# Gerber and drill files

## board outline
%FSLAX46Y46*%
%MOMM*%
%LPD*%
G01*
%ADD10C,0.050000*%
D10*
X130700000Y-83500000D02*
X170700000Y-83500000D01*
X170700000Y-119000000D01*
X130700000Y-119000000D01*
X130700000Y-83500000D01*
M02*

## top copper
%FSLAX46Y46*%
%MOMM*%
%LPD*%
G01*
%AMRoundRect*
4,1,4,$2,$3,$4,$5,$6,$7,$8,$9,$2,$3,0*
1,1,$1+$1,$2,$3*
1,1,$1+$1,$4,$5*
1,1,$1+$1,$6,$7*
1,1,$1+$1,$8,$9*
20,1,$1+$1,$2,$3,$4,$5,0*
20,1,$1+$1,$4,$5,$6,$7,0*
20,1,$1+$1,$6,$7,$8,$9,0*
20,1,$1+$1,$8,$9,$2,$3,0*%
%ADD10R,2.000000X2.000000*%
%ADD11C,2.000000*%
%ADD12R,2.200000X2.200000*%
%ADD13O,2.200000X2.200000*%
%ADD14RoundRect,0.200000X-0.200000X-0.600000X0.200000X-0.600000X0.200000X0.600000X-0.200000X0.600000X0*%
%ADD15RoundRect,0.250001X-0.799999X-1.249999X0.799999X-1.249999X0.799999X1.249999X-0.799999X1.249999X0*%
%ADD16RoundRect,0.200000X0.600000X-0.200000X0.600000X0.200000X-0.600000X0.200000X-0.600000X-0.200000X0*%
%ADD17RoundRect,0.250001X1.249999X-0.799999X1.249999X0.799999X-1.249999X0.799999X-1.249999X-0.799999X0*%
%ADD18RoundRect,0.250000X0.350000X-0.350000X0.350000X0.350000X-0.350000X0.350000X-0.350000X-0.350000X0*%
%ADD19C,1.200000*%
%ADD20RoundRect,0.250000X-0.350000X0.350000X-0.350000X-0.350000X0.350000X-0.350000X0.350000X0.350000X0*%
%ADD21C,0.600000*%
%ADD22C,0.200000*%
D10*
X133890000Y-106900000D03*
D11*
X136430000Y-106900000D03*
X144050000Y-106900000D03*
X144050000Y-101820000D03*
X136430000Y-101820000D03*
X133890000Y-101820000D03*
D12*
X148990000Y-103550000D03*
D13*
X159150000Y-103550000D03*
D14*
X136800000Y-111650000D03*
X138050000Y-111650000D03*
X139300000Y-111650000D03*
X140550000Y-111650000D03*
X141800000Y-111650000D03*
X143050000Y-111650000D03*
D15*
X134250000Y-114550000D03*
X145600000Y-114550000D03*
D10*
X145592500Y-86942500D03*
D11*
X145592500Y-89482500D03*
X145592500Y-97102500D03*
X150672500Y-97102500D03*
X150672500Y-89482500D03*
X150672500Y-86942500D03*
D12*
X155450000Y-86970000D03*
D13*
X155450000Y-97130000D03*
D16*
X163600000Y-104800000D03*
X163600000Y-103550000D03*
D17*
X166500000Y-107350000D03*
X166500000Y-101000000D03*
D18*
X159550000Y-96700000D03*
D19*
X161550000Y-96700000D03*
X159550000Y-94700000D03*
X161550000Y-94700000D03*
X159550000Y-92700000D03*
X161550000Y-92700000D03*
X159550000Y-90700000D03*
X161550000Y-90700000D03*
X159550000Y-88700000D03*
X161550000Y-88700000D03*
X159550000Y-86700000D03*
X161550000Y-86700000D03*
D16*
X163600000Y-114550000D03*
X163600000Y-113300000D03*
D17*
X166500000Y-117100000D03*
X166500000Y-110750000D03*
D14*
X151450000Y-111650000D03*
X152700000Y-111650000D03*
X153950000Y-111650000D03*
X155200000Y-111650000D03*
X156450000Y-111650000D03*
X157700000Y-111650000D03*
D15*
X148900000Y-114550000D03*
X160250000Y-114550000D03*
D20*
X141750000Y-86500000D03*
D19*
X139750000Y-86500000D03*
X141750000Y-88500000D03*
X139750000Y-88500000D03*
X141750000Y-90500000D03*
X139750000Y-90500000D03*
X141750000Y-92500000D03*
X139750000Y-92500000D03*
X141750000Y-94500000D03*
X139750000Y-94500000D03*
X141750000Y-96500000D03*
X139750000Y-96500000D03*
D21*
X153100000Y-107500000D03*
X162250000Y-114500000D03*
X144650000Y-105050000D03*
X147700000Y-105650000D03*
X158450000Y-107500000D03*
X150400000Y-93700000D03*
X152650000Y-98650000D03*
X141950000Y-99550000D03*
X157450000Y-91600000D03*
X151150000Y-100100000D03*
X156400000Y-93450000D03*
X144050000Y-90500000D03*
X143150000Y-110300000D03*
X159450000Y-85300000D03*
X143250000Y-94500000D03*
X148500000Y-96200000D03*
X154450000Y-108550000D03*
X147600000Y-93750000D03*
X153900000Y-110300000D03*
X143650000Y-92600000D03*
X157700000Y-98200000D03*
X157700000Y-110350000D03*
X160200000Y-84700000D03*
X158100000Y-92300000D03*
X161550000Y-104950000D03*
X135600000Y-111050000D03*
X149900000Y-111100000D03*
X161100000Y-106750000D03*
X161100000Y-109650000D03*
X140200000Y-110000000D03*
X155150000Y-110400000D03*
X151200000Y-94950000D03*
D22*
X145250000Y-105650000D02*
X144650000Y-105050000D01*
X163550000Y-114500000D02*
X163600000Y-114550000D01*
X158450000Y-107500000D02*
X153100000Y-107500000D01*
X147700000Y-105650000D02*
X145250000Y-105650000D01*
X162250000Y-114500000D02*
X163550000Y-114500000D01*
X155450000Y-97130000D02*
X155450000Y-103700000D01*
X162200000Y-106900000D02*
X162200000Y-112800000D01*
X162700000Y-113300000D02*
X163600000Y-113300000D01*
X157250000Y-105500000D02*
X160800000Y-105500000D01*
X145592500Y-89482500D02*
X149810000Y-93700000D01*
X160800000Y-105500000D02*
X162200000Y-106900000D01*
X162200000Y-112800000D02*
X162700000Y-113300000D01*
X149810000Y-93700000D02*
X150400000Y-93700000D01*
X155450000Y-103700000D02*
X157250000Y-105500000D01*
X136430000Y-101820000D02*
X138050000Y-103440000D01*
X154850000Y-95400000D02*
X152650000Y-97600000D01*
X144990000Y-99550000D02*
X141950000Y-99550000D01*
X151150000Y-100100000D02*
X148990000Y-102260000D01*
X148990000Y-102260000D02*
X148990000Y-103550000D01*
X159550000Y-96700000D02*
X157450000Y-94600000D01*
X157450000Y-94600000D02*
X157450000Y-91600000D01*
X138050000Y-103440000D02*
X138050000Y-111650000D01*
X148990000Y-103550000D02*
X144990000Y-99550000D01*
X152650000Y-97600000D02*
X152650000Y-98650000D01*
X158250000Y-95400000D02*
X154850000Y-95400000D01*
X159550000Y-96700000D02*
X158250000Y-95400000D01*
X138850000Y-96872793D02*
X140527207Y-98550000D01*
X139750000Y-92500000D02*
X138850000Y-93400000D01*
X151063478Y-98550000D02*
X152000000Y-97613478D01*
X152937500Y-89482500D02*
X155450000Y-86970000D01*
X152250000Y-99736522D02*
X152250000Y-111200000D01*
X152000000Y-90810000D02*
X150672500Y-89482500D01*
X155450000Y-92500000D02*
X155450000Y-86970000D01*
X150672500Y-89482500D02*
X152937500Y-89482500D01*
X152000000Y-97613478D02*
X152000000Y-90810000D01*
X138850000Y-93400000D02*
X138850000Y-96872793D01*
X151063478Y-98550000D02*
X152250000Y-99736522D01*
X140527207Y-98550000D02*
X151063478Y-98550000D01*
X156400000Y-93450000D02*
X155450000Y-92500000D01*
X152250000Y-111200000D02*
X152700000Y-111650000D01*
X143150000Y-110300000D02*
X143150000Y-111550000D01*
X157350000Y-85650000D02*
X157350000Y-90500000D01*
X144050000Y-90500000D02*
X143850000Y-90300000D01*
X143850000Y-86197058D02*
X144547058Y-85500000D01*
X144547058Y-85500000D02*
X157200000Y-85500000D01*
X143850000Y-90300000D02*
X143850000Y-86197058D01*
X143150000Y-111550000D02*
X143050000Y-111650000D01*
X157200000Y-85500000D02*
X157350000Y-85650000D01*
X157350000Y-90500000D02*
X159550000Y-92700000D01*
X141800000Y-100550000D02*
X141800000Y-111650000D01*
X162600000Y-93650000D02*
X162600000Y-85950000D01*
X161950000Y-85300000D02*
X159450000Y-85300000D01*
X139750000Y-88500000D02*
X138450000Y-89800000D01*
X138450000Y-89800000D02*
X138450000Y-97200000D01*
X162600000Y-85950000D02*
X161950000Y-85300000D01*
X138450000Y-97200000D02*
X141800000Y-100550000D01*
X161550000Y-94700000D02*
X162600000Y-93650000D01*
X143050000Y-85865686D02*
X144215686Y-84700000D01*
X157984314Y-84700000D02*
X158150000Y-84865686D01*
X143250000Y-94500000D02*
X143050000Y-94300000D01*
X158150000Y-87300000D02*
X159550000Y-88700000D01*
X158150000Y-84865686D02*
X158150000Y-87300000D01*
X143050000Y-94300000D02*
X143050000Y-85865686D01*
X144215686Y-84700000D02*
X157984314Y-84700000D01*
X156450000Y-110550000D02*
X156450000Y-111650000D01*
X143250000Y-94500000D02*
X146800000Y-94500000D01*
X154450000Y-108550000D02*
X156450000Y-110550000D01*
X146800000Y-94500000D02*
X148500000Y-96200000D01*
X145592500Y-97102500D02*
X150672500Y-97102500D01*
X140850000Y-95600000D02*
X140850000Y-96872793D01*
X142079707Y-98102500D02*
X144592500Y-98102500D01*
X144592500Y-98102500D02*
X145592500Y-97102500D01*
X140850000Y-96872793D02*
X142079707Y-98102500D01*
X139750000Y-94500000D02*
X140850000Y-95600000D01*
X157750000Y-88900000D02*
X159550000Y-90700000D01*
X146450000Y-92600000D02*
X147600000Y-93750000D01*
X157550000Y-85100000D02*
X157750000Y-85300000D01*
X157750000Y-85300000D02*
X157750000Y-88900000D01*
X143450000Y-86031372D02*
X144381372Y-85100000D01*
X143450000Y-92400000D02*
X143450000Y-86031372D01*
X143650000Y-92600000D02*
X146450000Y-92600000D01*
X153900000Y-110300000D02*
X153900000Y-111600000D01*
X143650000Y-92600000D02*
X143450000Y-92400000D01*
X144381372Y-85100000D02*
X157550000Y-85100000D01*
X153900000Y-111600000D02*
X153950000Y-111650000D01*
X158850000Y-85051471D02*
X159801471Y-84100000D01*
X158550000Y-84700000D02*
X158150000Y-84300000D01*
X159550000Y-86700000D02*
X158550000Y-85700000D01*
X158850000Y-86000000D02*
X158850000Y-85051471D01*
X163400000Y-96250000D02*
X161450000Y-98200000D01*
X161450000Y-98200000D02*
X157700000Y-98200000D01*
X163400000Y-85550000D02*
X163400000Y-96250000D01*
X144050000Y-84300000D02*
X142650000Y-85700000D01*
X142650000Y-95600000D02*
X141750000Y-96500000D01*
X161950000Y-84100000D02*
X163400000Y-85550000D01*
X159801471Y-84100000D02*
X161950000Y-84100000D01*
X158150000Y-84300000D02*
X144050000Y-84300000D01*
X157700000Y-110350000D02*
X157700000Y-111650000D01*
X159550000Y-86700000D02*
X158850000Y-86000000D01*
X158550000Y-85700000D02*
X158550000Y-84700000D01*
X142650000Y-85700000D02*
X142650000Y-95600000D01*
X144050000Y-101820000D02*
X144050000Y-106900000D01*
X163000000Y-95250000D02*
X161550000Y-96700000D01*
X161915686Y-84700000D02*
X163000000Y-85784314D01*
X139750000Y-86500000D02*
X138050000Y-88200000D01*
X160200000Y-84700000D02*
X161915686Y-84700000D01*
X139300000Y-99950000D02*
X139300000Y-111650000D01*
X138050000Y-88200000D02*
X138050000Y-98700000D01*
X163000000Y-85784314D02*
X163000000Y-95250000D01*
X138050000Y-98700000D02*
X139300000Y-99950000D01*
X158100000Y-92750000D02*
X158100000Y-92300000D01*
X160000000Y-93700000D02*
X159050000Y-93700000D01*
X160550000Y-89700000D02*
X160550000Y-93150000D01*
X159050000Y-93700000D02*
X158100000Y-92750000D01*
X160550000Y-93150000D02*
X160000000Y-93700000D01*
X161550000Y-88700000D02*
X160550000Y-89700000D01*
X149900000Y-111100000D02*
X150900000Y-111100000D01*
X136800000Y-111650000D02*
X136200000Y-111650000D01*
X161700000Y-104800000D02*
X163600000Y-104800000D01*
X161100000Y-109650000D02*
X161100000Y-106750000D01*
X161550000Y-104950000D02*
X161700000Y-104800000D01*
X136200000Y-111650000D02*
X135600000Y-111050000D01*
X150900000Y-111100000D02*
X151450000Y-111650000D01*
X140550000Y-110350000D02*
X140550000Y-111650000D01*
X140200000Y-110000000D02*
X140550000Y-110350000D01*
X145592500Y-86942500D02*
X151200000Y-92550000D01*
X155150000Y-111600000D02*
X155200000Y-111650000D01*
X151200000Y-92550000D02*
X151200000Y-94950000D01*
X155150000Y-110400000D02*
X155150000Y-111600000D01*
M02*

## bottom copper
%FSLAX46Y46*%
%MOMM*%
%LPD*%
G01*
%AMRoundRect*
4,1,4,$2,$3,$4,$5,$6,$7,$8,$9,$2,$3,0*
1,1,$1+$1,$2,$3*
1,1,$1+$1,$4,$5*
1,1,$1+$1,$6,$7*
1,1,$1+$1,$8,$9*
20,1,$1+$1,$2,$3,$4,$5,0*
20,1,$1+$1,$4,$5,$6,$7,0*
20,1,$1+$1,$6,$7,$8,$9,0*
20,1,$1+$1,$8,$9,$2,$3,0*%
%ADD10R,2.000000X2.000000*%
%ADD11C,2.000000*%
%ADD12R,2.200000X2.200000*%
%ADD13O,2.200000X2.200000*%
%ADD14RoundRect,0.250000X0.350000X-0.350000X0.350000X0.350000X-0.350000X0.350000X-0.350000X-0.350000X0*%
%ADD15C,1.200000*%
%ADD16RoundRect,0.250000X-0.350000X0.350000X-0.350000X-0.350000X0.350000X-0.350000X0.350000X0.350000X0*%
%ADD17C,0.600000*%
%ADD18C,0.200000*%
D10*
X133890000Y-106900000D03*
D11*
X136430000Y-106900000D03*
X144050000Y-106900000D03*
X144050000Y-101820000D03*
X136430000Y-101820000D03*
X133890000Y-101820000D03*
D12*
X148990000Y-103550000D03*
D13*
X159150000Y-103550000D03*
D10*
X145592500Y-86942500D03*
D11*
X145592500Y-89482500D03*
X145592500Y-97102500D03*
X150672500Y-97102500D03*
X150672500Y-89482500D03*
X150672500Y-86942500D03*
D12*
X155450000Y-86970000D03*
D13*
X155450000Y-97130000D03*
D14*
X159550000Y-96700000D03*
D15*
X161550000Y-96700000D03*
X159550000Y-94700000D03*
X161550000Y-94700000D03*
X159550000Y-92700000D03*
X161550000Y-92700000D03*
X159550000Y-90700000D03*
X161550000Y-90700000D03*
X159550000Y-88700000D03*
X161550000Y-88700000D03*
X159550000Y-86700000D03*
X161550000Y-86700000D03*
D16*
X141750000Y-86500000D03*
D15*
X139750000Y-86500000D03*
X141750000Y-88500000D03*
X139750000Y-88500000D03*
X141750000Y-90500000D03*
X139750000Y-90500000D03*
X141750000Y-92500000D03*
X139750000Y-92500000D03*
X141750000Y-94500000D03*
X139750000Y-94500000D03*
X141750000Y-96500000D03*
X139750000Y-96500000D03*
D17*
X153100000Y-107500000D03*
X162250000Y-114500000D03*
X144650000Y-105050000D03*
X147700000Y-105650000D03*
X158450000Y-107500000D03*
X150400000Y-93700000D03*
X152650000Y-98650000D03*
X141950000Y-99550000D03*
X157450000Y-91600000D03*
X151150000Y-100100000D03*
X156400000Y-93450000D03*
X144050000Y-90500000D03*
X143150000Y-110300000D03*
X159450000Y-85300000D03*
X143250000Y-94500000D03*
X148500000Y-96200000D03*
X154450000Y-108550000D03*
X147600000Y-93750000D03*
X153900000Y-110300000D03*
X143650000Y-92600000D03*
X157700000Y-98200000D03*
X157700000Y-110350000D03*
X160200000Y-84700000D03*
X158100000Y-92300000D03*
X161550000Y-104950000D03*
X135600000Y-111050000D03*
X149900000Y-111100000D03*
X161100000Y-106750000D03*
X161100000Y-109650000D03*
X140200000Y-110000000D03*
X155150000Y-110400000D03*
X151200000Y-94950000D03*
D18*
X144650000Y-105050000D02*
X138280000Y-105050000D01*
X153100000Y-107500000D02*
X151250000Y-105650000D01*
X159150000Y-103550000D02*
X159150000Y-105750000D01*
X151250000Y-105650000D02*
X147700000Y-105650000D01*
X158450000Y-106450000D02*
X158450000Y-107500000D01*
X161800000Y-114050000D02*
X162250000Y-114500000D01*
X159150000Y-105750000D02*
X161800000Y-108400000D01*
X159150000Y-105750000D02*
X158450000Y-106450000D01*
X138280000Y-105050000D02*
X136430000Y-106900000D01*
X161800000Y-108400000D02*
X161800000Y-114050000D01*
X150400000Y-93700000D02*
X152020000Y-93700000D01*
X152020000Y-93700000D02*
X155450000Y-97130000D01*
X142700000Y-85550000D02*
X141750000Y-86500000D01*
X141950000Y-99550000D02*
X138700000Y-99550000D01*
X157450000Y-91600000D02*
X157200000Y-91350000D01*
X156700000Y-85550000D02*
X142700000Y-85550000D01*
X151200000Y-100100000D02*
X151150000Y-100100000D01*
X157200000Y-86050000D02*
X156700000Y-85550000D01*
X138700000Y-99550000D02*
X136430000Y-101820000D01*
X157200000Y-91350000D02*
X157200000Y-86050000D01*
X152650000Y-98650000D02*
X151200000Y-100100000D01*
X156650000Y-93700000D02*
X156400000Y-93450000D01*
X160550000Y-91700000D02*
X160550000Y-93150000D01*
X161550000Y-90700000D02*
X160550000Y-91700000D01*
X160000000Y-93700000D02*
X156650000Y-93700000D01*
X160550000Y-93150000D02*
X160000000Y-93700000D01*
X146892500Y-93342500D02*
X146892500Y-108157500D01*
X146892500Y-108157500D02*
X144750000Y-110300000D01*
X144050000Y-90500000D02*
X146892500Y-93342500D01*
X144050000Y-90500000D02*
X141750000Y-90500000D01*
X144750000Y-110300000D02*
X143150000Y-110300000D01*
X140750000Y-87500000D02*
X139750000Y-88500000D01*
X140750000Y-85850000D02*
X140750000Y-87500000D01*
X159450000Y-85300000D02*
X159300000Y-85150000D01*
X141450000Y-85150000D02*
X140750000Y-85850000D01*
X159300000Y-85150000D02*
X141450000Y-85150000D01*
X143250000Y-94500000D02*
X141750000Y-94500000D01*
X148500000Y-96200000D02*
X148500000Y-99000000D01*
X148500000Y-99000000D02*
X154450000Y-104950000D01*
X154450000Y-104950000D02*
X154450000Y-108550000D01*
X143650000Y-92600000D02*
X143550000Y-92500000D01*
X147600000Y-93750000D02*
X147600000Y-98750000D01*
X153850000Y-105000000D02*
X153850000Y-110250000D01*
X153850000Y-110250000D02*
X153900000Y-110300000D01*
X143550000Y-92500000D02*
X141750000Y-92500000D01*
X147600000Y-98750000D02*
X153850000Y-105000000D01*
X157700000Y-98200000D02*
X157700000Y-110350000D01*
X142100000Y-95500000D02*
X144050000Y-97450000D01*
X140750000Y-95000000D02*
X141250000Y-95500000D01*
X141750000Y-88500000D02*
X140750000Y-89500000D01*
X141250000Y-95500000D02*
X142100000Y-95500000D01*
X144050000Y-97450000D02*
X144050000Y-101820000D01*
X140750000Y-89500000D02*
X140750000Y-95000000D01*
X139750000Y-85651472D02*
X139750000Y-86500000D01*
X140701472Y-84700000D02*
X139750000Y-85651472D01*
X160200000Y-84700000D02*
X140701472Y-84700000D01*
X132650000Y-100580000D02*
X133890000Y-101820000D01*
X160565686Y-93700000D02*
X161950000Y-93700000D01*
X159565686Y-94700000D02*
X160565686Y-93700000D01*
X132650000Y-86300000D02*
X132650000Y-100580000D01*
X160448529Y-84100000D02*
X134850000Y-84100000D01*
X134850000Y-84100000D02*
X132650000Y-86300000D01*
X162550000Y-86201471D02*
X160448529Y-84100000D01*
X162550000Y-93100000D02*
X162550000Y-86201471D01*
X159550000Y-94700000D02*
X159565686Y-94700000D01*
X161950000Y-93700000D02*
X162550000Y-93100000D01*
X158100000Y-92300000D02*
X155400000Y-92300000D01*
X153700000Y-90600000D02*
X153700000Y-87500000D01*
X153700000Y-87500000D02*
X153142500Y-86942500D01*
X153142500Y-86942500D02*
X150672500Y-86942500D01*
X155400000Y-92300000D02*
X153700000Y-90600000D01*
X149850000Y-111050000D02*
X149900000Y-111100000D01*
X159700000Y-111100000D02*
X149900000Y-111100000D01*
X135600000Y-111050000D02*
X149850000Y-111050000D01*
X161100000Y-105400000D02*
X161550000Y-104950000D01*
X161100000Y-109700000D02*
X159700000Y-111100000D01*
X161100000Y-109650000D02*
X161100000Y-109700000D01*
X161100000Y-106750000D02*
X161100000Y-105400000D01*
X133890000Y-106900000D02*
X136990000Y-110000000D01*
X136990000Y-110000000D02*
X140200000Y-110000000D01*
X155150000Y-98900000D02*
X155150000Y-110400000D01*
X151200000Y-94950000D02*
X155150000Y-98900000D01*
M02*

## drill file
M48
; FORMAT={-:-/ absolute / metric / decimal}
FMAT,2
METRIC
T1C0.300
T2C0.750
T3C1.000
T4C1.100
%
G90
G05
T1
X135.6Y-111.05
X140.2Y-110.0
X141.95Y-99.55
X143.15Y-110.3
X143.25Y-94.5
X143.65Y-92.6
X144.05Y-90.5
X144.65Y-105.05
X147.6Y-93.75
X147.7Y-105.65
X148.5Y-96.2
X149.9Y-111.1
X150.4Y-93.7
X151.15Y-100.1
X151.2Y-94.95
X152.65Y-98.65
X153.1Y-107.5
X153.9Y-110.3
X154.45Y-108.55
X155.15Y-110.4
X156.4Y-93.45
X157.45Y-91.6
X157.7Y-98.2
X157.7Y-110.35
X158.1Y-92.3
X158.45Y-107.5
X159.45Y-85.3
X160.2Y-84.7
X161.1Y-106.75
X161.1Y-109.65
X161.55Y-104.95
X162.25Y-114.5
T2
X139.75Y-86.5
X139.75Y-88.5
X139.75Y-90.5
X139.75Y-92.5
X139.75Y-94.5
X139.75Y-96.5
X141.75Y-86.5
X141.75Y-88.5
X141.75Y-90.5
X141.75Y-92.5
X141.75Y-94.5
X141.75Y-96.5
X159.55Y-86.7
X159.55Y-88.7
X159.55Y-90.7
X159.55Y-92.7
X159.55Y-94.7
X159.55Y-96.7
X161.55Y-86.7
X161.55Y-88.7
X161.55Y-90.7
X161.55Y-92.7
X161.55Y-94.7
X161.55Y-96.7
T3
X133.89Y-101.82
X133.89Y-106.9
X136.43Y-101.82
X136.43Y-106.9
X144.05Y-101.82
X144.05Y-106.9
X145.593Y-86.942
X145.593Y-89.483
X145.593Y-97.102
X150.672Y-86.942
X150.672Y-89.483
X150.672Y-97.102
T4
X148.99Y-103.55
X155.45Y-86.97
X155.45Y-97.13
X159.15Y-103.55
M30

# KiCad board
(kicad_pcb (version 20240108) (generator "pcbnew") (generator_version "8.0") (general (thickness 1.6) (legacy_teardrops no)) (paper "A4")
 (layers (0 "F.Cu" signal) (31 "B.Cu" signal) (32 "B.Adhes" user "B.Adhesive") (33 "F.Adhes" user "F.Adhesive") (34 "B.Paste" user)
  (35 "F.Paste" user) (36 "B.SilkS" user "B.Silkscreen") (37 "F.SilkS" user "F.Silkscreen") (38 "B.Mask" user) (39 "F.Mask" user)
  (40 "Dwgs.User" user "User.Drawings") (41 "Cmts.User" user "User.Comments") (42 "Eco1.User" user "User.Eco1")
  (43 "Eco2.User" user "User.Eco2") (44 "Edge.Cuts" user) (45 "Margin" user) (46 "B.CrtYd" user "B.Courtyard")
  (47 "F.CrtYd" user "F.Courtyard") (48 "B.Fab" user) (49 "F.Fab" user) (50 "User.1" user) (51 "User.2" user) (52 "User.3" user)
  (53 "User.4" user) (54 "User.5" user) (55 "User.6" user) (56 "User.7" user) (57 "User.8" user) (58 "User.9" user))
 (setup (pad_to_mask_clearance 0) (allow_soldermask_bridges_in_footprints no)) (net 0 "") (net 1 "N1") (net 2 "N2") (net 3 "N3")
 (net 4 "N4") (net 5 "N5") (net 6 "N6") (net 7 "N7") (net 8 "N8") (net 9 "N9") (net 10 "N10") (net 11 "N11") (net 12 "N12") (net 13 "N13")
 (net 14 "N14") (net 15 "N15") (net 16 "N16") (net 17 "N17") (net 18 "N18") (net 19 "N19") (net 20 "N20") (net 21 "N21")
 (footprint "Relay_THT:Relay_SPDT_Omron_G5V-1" (layer "F.Cu") (at 133.89 106.9 90)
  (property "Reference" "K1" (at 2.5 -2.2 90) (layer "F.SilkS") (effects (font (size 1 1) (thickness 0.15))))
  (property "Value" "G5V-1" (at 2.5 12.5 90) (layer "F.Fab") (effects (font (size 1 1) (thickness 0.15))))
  (pad "1" thru_hole rect (at 0 0 90) (size 2 2) (drill 1) (layers "*.Cu" "*.Mask") (remove_unused_layers no) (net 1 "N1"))
  (pad "2" thru_hole circle (at 0 2.54 90) (size 2 2) (drill 1) (layers "*.Cu" "*.Mask") (remove_unused_layers no) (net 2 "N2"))
  (pad "5" thru_hole circle (at 0 10.16 90) (size 2 2) (drill 1) (layers "*.Cu" "*.Mask") (remove_unused_layers no) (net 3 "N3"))
  (pad "6" thru_hole circle (at 5.08 10.16 90) (size 2 2) (drill 1) (layers "*.Cu" "*.Mask") (remove_unused_layers no) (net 3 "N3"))
  (pad "9" thru_hole circle (at 5.08 2.54 90) (size 2 2) (drill 1) (layers "*.Cu" "*.Mask") (remove_unused_layers no) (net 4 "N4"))
  (pad "10" thru_hole circle (at 5.08 0 90) (size 2 2) (drill 1) (layers "*.Cu" "*.Mask") (remove_unused_layers no) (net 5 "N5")))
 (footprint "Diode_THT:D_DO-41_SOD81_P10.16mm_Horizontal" (layer "F.Cu") (at 148.99 103.55)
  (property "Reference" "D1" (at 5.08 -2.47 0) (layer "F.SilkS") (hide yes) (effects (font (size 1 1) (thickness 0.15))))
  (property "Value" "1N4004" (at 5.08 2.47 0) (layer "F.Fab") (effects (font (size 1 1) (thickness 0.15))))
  (pad "1" thru_hole rect (at 0 0) (size 2.2 2.2) (drill 1.1) (layers "*.Cu" "*.Mask") (remove_unused_layers no) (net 4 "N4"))
  (pad "2" thru_hole oval (at 10.16 0) (size 2.2 2.2) (drill 1.1) (layers "*.Cu" "*.Mask") (remove_unused_layers no) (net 2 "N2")))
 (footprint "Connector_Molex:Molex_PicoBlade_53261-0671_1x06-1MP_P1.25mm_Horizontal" (layer "F.Cu") (at 139.925 114.05)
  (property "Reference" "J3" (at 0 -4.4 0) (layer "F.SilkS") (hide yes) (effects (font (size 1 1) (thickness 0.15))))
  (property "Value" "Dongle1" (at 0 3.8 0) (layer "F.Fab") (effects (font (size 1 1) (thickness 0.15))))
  (pad "1" smd roundrect (at -3.125 -2.4) (size 0.8 1.6) (layers "F.Cu" "F.Paste" "F.Mask") (roundrect_rratio 0.25) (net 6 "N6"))
  (pad "2" smd roundrect (at -1.875 -2.4) (size 0.8 1.6) (layers "F.Cu" "F.Paste" "F.Mask") (roundrect_rratio 0.25) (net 4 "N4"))
  (pad "3" smd roundrect (at -0.625 -2.4) (size 0.8 1.6) (layers "F.Cu" "F.Paste" "F.Mask") (roundrect_rratio 0.25) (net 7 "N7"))
  (pad "4" smd roundrect (at 0.625 -2.4) (size 0.8 1.6) (layers "F.Cu" "F.Paste" "F.Mask") (roundrect_rratio 0.25) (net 1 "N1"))
  (pad "5" smd roundrect (at 1.875 -2.4) (size 0.8 1.6) (layers "F.Cu" "F.Paste" "F.Mask") (roundrect_rratio 0.25) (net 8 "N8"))
  (pad "6" smd roundrect (at 3.125 -2.4) (size 0.8 1.6) (layers "F.Cu" "F.Paste" "F.Mask") (roundrect_rratio 0.25) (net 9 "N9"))
  (pad "MP" smd roundrect (at -5.675 0.5) (size 2.1 3) (layers "F.Cu" "F.Paste" "F.Mask") (roundrect_rratio 0.119048))
  (pad "MP" smd roundrect (at 5.675 0.5) (size 2.1 3) (layers "F.Cu" "F.Paste" "F.Mask") (roundrect_rratio 0.119048)))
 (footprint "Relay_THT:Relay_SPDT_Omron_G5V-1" (layer "F.Cu") (at 145.5925 86.9425)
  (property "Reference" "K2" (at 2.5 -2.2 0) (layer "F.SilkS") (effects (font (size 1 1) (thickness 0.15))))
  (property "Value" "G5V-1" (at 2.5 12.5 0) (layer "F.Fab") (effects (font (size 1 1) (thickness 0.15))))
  (pad "1" thru_hole rect (at 0 0) (size 2 2) (drill 1) (layers "*.Cu" "*.Mask") (remove_unused_layers no) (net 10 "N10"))
  (pad "2" thru_hole circle (at 0 2.54) (size 2 2) (drill 1) (layers "*.Cu" "*.Mask") (remove_unused_layers no) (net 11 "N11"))
  (pad "5" thru_hole circle (at 0 10.16) (size 2 2) (drill 1) (layers "*.Cu" "*.Mask") (remove_unused_layers no) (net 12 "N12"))
  (pad "6" thru_hole circle (at 5.08 10.16) (size 2 2) (drill 1) (layers "*.Cu" "*.Mask") (remove_unused_layers no) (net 12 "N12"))
  (pad "9" thru_hole circle (at 5.08 2.54) (size 2 2) (drill 1) (layers "*.Cu" "*.Mask") (remove_unused_layers no) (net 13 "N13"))
  (pad "10" thru_hole circle (at 5.08 0) (size 2 2) (drill 1) (layers "*.Cu" "*.Mask") (remove_unused_layers no) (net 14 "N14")))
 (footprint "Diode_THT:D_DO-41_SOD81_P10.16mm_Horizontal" (layer "F.Cu") (at 155.45 86.97 -90)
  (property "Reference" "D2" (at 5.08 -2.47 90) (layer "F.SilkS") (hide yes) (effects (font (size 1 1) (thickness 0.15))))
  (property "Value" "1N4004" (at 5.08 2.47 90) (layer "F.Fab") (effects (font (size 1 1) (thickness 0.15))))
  (pad "1" thru_hole rect (at 0 0 270) (size 2.2 2.2) (drill 1.1) (layers "*.Cu" "*.Mask") (remove_unused_layers no) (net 13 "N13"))
  (pad "2" thru_hole oval (at 10.16 0 270) (size 2.2 2.2) (drill 1.1) (layers "*.Cu" "*.Mask") (remove_unused_layers no) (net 11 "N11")))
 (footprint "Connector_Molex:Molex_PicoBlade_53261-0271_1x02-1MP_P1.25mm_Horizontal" (layer "F.Cu") (at 166 104.175 90)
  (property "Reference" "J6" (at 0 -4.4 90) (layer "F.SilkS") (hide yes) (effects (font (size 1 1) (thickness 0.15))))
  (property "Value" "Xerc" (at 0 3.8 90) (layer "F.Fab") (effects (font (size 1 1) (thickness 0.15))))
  (pad "1" smd roundrect (at -0.625 -2.4 90) (size 0.8 1.6) (layers "F.Cu" "F.Paste" "F.Mask") (roundrect_rratio 0.25) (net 6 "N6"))
  (pad "2" smd roundrect (at 0.625 -2.4 90) (size 0.8 1.6) (layers "F.Cu" "F.Paste" "F.Mask") (roundrect_rratio 0.25))
  (pad "MP" smd roundrect (at -3.175 0.5 90) (size 2.1 3) (layers "F.Cu" "F.Paste" "F.Mask") (roundrect_rratio 0.119048))
  (pad "MP" smd roundrect (at 3.175 0.5 90) (size 2.1 3) (layers "F.Cu" "F.Paste" "F.Mask") (roundrect_rratio 0.119048)))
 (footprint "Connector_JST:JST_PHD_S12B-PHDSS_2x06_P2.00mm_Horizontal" (layer "F.Cu") (at 159.55 96.7 90)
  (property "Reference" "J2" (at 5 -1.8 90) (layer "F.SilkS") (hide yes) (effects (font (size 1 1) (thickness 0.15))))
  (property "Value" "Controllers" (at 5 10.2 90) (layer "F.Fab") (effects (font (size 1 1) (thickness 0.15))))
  (pad "1" thru_hole roundrect (at 0 0 90) (size 1.2 1.2) (drill 0.75) (layers "*.Cu" "*.Mask") (remove_unused_layers no)
   (roundrect_rratio 0.208333) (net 4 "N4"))
  (pad "2" thru_hole circle (at 0 2 90) (size 1.2 1.2) (drill 0.75) (layers "*.Cu" "*.Mask") (remove_unused_layers no) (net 7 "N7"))
  (pad "3" thru_hole circle (at 2 0 90) (size 1.2 1.2) (drill 0.75) (layers "*.Cu" "*.Mask") (remove_unused_layers no) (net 5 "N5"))
  (pad "4" thru_hole circle (at 2 2 90) (size 1.2 1.2) (drill 0.75) (layers "*.Cu" "*.Mask") (remove_unused_layers no) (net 8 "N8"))
  (pad "5" thru_hole circle (at 4 0 90) (size 1.2 1.2) (drill 0.75) (layers "*.Cu" "*.Mask") (remove_unused_layers no) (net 9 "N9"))
  (pad "6" thru_hole circle (at 4 2 90) (size 1.2 1.2) (drill 0.75) (layers "*.Cu" "*.Mask") (remove_unused_layers no) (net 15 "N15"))
  (pad "7" thru_hole circle (at 6 0 90) (size 1.2 1.2) (drill 0.75) (layers "*.Cu" "*.Mask") (remove_unused_layers no) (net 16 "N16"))
  (pad "8" thru_hole circle (at 6 2 90) (size 1.2 1.2) (drill 0.75) (layers "*.Cu" "*.Mask") (remove_unused_layers no) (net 13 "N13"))
  (pad "9" thru_hole circle (at 8 0 90) (size 1.2 1.2) (drill 0.75) (layers "*.Cu" "*.Mask") (remove_unused_layers no) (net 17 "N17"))
  (pad "10" thru_hole circle (at 8 2 90) (size 1.2 1.2) (drill 0.75) (layers "*.Cu" "*.Mask") (remove_unused_layers no) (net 14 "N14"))
  (pad "11" thru_hole circle (at 10 0 90) (size 1.2 1.2) (drill 0.75) (layers "*.Cu" "*.Mask") (remove_unused_layers no) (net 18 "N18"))
  (pad "12" thru_hole circle (at 10 2 90) (size 1.2 1.2) (drill 0.75) (layers "*.Cu" "*.Mask") (remove_unused_layers no) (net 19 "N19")))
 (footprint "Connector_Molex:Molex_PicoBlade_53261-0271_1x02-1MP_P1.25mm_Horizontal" (layer "F.Cu") (at 166 113.925 90)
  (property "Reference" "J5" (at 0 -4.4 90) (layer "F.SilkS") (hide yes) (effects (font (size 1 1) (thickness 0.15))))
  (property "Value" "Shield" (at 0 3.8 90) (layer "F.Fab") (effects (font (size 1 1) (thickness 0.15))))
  (pad "1" smd roundrect (at -0.625 -2.4 90) (size 0.8 1.6) (layers "F.Cu" "F.Paste" "F.Mask") (roundrect_rratio 0.25) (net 2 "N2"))
  (pad "2" smd roundrect (at 0.625 -2.4 90) (size 0.8 1.6) (layers "F.Cu" "F.Paste" "F.Mask") (roundrect_rratio 0.25) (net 11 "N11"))
  (pad "MP" smd roundrect (at -3.175 0.5 90) (size 2.1 3) (layers "F.Cu" "F.Paste" "F.Mask") (roundrect_rratio 0.119048))
  (pad "MP" smd roundrect (at 3.175 0.5 90) (size 2.1 3) (layers "F.Cu" "F.Paste" "F.Mask") (roundrect_rratio 0.119048)))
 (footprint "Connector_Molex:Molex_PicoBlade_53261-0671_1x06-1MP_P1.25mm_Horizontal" (layer "F.Cu") (at 154.575 114.05)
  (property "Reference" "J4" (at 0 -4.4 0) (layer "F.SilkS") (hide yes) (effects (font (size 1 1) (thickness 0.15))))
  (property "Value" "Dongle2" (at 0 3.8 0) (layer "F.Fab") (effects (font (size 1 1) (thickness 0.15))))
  (pad "1" smd roundrect (at -3.125 -2.4) (size 0.8 1.6) (layers "F.Cu" "F.Paste" "F.Mask") (roundrect_rratio 0.25) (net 6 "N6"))
  (pad "2" smd roundrect (at -1.875 -2.4) (size 0.8 1.6) (layers "F.Cu" "F.Paste" "F.Mask") (roundrect_rratio 0.25) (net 13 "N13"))
  (pad "3" smd roundrect (at -0.625 -2.4) (size 0.8 1.6) (layers "F.Cu" "F.Paste" "F.Mask") (roundrect_rratio 0.25) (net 16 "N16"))
  (pad "4" smd roundrect (at 0.625 -2.4) (size 0.8 1.6) (layers "F.Cu" "F.Paste" "F.Mask") (roundrect_rratio 0.25) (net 10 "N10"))
  (pad "5" smd roundrect (at 1.875 -2.4) (size 0.8 1.6) (layers "F.Cu" "F.Paste" "F.Mask") (roundrect_rratio 0.25) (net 17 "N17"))
  (pad "6" smd roundrect (at 3.125 -2.4) (size 0.8 1.6) (layers "F.Cu" "F.Paste" "F.Mask") (roundrect_rratio 0.25) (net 18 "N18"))
  (pad "MP" smd roundrect (at -5.675 0.5) (size 2.1 3) (layers "F.Cu" "F.Paste" "F.Mask") (roundrect_rratio 0.119048))
  (pad "MP" smd roundrect (at 5.675 0.5) (size 2.1 3) (layers "F.Cu" "F.Paste" "F.Mask") (roundrect_rratio 0.119048)))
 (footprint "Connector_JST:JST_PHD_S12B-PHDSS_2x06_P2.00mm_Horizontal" (layer "F.Cu") (at 141.75 86.5 -90)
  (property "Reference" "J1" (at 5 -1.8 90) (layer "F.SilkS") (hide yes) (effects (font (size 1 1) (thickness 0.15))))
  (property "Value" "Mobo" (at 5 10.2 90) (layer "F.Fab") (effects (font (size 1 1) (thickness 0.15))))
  (pad "1" thru_hole roundrect (at 0 0 270) (size 1.2 1.2) (drill 0.75) (layers "*.Cu" "*.Mask") (remove_unused_layers no)
   (roundrect_rratio 0.208333) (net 4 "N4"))
  (pad "2" thru_hole circle (at 0 2 270) (size 1.2 1.2) (drill 0.75) (layers "*.Cu" "*.Mask") (remove_unused_layers no) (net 7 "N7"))
  (pad "3" thru_hole circle (at 2 0 270) (size 1.2 1.2) (drill 0.75) (layers "*.Cu" "*.Mask") (remove_unused_layers no) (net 3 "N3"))
  (pad "4" thru_hole circle (at 2 2 270) (size 1.2 1.2) (drill 0.75) (layers "*.Cu" "*.Mask") (remove_unused_layers no) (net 8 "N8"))
  (pad "5" thru_hole circle (at 4 0 270) (size 1.2 1.2) (drill 0.75) (layers "*.Cu" "*.Mask") (remove_unused_layers no) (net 9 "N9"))
  (pad "6" thru_hole circle (at 4 2 270) (size 1.2 1.2) (drill 0.75) (layers "*.Cu" "*.Mask") (remove_unused_layers no) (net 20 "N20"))
  (pad "7" thru_hole circle (at 6 0 270) (size 1.2 1.2) (drill 0.75) (layers "*.Cu" "*.Mask") (remove_unused_layers no) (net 16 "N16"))
  (pad "8" thru_hole circle (at 6 2 270) (size 1.2 1.2) (drill 0.75) (layers "*.Cu" "*.Mask") (remove_unused_layers no) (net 13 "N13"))
  (pad "9" thru_hole circle (at 8 0 270) (size 1.2 1.2) (drill 0.75) (layers "*.Cu" "*.Mask") (remove_unused_layers no) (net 17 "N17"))
  (pad "10" thru_hole circle (at 8 2 270) (size 1.2 1.2) (drill 0.75) (layers "*.Cu" "*.Mask") (remove_unused_layers no) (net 12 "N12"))
  (pad "11" thru_hole circle (at 10 0 270) (size 1.2 1.2) (drill 0.75) (layers "*.Cu" "*.Mask") (remove_unused_layers no) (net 18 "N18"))
  (pad "12" thru_hole circle (at 10 2 270) (size 1.2 1.2) (drill 0.75) (layers "*.Cu" "*.Mask") (remove_unused_layers no) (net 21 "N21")))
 (gr_rect (start 130.7 83.5) (end 170.7 119) (stroke (width 0.05) (type default)) (fill none) (layer "Edge.Cuts"))
 (segment (start 145.25 105.65) (end 144.65 105.05) (width 0.2) (layer "F.Cu") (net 2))
 (segment (start 163.55 114.5) (end 163.6 114.55) (width 0.2) (layer "F.Cu") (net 2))
 (segment (start 158.45 107.5) (end 153.1 107.5) (width 0.2) (layer "F.Cu") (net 2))
 (segment (start 147.7 105.65) (end 145.25 105.65) (width 0.2) (layer "F.Cu") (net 2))
 (segment (start 162.25 114.5) (end 163.55 114.5) (width 0.2) (layer "F.Cu") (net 2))
 (via (at 153.1 107.5) (size 0.6) (drill 0.3) (layers "F.Cu" "B.Cu") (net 2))
 (via (at 162.25 114.5) (size 0.6) (drill 0.3) (layers "F.Cu" "B.Cu") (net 2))
 (via (at 144.65 105.05) (size 0.6) (drill 0.3) (layers "F.Cu" "B.Cu") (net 2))
 (via (at 147.7 105.65) (size 0.6) (drill 0.3) (layers "F.Cu" "B.Cu") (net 2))
 (via (at 158.45 107.5) (size 0.6) (drill 0.3) (layers "F.Cu" "B.Cu") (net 2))
 (segment (start 144.65 105.05) (end 138.28 105.05) (width 0.2) (layer "B.Cu") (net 2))
 (segment (start 153.1 107.5) (end 151.25 105.65) (width 0.2) (layer "B.Cu") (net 2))
 (segment (start 159.15 103.55) (end 159.15 105.75) (width 0.2) (layer "B.Cu") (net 2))
 (segment (start 151.25 105.65) (end 147.7 105.65) (width 0.2) (layer "B.Cu") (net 2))
 (segment (start 158.45 106.45) (end 158.45 107.5) (width 0.2) (layer "B.Cu") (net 2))
 (segment (start 161.8 114.05) (end 162.25 114.5) (width 0.2) (layer "B.Cu") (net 2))
 (segment (start 159.15 105.75) (end 161.8 108.4) (width 0.2) (layer "B.Cu") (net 2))
 (segment (start 159.15 105.75) (end 158.45 106.45) (width 0.2) (layer "B.Cu") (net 2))
 (segment (start 138.28 105.05) (end 136.43 106.9) (width 0.2) (layer "B.Cu") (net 2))
 (segment (start 161.8 108.4) (end 161.8 114.05) (width 0.2) (layer "B.Cu") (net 2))
 (segment (start 155.45 97.13) (end 155.45 103.7) (width 0.2) (layer "F.Cu") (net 11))
 (segment (start 162.2 106.9) (end 162.2 112.8) (width 0.2) (layer "F.Cu") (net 11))
 (segment (start 162.7 113.3) (end 163.6 113.3) (width 0.2) (layer "F.Cu") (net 11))
 (segment (start 157.25 105.5) (end 160.8 105.5) (width 0.2) (layer "F.Cu") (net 11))
 (segment (start 145.5925 89.4825) (end 149.81 93.7) (width 0.2) (layer "F.Cu") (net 11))
 (segment (start 160.8 105.5) (end 162.2 106.9) (width 0.2) (layer "F.Cu") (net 11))
 (segment (start 162.2 112.8) (end 162.7 113.3) (width 0.2) (layer "F.Cu") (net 11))
 (segment (start 149.81 93.7) (end 150.4 93.7) (width 0.2) (layer "F.Cu") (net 11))
 (segment (start 155.45 103.7) (end 157.25 105.5) (width 0.2) (layer "F.Cu") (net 11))
 (via (at 150.4 93.7) (size 0.6) (drill 0.3) (layers "F.Cu" "B.Cu") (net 11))
 (segment (start 150.4 93.7) (end 152.02 93.7) (width 0.2) (layer "B.Cu") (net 11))
 (segment (start 152.02 93.7) (end 155.45 97.13) (width 0.2) (layer "B.Cu") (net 11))
 (segment (start 136.43 101.82) (end 138.05 103.44) (width 0.2) (layer "F.Cu") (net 4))
 (segment (start 154.85 95.4) (end 152.65 97.6) (width 0.2) (layer "F.Cu") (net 4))
 (segment (start 144.99 99.55) (end 141.95 99.55) (width 0.2) (layer "F.Cu") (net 4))
 (segment (start 151.15 100.1) (end 148.99 102.26) (width 0.2) (layer "F.Cu") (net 4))
 (segment (start 148.99 102.26) (end 148.99 103.55) (width 0.2) (layer "F.Cu") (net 4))
 (segment (start 159.55 96.7) (end 157.45 94.6) (width 0.2) (layer "F.Cu") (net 4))
 (segment (start 157.45 94.6) (end 157.45 91.6) (width 0.2) (layer "F.Cu") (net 4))
 (segment (start 138.05 103.44) (end 138.05 111.65) (width 0.2) (layer "F.Cu") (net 4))
 (segment (start 148.99 103.55) (end 144.99 99.55) (width 0.2) (layer "F.Cu") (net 4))
 (segment (start 152.65 97.6) (end 152.65 98.65) (width 0.2) (layer "F.Cu") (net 4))
 (segment (start 158.25 95.4) (end 154.85 95.4) (width 0.2) (layer "F.Cu") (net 4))
 (segment (start 159.55 96.7) (end 158.25 95.4) (width 0.2) (layer "F.Cu") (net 4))
 (via (at 152.65 98.65) (size 0.6) (drill 0.3) (layers "F.Cu" "B.Cu") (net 4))
 (via (at 141.95 99.55) (size 0.6) (drill 0.3) (layers "F.Cu" "B.Cu") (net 4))
 (via (at 157.45 91.6) (size 0.6) (drill 0.3) (layers "F.Cu" "B.Cu") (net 4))
 (via (at 151.15 100.1) (size 0.6) (drill 0.3) (layers "F.Cu" "B.Cu") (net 4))
 (segment (start 142.7 85.55) (end 141.75 86.5) (width 0.2) (layer "B.Cu") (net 4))
 (segment (start 141.95 99.55) (end 138.7 99.55) (width 0.2) (layer "B.Cu") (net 4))
 (segment (start 157.45 91.6) (end 157.2 91.35) (width 0.2) (layer "B.Cu") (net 4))
 (segment (start 156.7 85.55) (end 142.7 85.55) (width 0.2) (layer "B.Cu") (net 4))
 (segment (start 151.2 100.1) (end 151.15 100.1) (width 0.2) (layer "B.Cu") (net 4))
 (segment (start 157.2 86.05) (end 156.7 85.55) (width 0.2) (layer "B.Cu") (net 4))
 (segment (start 138.7 99.55) (end 136.43 101.82) (width 0.2) (layer "B.Cu") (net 4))
 (segment (start 157.2 91.35) (end 157.2 86.05) (width 0.2) (layer "B.Cu") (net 4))
 (segment (start 152.65 98.65) (end 151.2 100.1) (width 0.2) (layer "B.Cu") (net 4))
 (segment (start 138.85 96.872793) (end 140.527207 98.55) (width 0.2) (layer "F.Cu") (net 13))
 (segment (start 139.75 92.5) (end 138.85 93.4) (width 0.2) (layer "F.Cu") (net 13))
 (segment (start 151.063478 98.55) (end 152 97.613478) (width 0.2) (layer "F.Cu") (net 13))
 (segment (start 152.9375 89.4825) (end 155.45 86.97) (width 0.2) (layer "F.Cu") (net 13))
 (segment (start 152.25 99.736522) (end 152.25 111.2) (width 0.2) (layer "F.Cu") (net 13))
 (segment (start 152 90.81) (end 150.6725 89.4825) (width 0.2) (layer "F.Cu") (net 13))
 (segment (start 155.45 92.5) (end 155.45 86.97) (width 0.2) (layer "F.Cu") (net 13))
 (segment (start 150.6725 89.4825) (end 152.9375 89.4825) (width 0.2) (layer "F.Cu") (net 13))
 (segment (start 152 97.613478) (end 152 90.81) (width 0.2) (layer "F.Cu") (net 13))
 (segment (start 138.85 93.4) (end 138.85 96.872793) (width 0.2) (layer "F.Cu") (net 13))
 (segment (start 151.063478 98.55) (end 152.25 99.736522) (width 0.2) (layer "F.Cu") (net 13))
 (segment (start 140.527207 98.55) (end 151.063478 98.55) (width 0.2) (layer "F.Cu") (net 13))
 (segment (start 156.4 93.45) (end 155.45 92.5) (width 0.2) (layer "F.Cu") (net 13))
 (segment (start 152.25 111.2) (end 152.7 111.65) (width 0.2) (layer "F.Cu") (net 13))
 (via (at 156.4 93.45) (size 0.6) (drill 0.3) (layers "F.Cu" "B.Cu") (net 13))
 (segment (start 156.65 93.7) (end 156.4 93.45) (width 0.2) (layer "B.Cu") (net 13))
 (segment (start 160.55 91.7) (end 160.55 93.15) (width 0.2) (layer "B.Cu") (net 13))
 (segment (start 161.55 90.7) (end 160.55 91.7) (width 0.2) (layer "B.Cu") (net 13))
 (segment (start 160 93.7) (end 156.65 93.7) (width 0.2) (layer "B.Cu") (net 13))
 (segment (start 160.55 93.15) (end 160 93.7) (width 0.2) (layer "B.Cu") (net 13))
 (segment (start 143.15 110.3) (end 143.15 111.55) (width 0.2) (layer "F.Cu") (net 9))
 (segment (start 157.35 85.65) (end 157.35 90.5) (width 0.2) (layer "F.Cu") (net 9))
 (segment (start 144.05 90.5) (end 143.85 90.3) (width 0.2) (layer "F.Cu") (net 9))
 (segment (start 143.85 86.197058) (end 144.547058 85.5) (width 0.2) (layer "F.Cu") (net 9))
 (segment (start 144.547058 85.5) (end 157.2 85.5) (width 0.2) (layer "F.Cu") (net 9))
 (segment (start 143.85 90.3) (end 143.85 86.197058) (width 0.2) (layer "F.Cu") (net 9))
 (segment (start 143.15 111.55) (end 143.05 111.65) (width 0.2) (layer "F.Cu") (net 9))
 (segment (start 157.2 85.5) (end 157.35 85.65) (width 0.2) (layer "F.Cu") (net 9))
 (segment (start 157.35 90.5) (end 159.55 92.7) (width 0.2) (layer "F.Cu") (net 9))
 (via (at 144.05 90.5) (size 0.6) (drill 0.3) (layers "F.Cu" "B.Cu") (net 9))
 (via (at 143.15 110.3) (size 0.6) (drill 0.3) (layers "F.Cu" "B.Cu") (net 9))
 (segment (start 146.8925 93.3425) (end 146.8925 108.1575) (width 0.2) (layer "B.Cu") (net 9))
 (segment (start 146.8925 108.1575) (end 144.75 110.3) (width 0.2) (layer "B.Cu") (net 9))
 (segment (start 144.05 90.5) (end 146.8925 93.3425) (width 0.2) (layer "B.Cu") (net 9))
 (segment (start 144.05 90.5) (end 141.75 90.5) (width 0.2) (layer "B.Cu") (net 9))
 (segment (start 144.75 110.3) (end 143.15 110.3) (width 0.2) (layer "B.Cu") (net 9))
 (segment (start 141.8 100.55) (end 141.8 111.65) (width 0.2) (layer "F.Cu") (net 8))
 (segment (start 162.6 93.65) (end 162.6 85.95) (width 0.2) (layer "F.Cu") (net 8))
 (segment (start 161.95 85.3) (end 159.45 85.3) (width 0.2) (layer "F.Cu") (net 8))
 (segment (start 139.75 88.5) (end 138.45 89.8) (width 0.2) (layer "F.Cu") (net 8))
 (segment (start 138.45 89.8) (end 138.45 97.2) (width 0.2) (layer "F.Cu") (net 8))
 (segment (start 162.6 85.95) (end 161.95 85.3) (width 0.2) (layer "F.Cu") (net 8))
 (segment (start 138.45 97.2) (end 141.8 100.55) (width 0.2) (layer "F.Cu") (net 8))
 (segment (start 161.55 94.7) (end 162.6 93.65) (width 0.2) (layer "F.Cu") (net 8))
 (via (at 159.45 85.3) (size 0.6) (drill 0.3) (layers "F.Cu" "B.Cu") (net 8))
 (segment (start 140.75 87.5) (end 139.75 88.5) (width 0.2) (layer "B.Cu") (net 8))
 (segment (start 140.75 85.85) (end 140.75 87.5) (width 0.2) (layer "B.Cu") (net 8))
 (segment (start 159.45 85.3) (end 159.3 85.15) (width 0.2) (layer "B.Cu") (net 8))
 (segment (start 141.45 85.15) (end 140.75 85.85) (width 0.2) (layer "B.Cu") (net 8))
 (segment (start 159.3 85.15) (end 141.45 85.15) (width 0.2) (layer "B.Cu") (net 8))
 (segment (start 143.05 85.865686) (end 144.215686 84.7) (width 0.2) (layer "F.Cu") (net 17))
 (segment (start 157.984314 84.7) (end 158.15 84.865686) (width 0.2) (layer "F.Cu") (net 17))
 (segment (start 143.25 94.5) (end 143.05 94.3) (width 0.2) (layer "F.Cu") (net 17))
 (segment (start 158.15 87.3) (end 159.55 88.7) (width 0.2) (layer "F.Cu") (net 17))
 (segment (start 158.15 84.865686) (end 158.15 87.3) (width 0.2) (layer "F.Cu") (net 17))
 (segment (start 143.05 94.3) (end 143.05 85.865686) (width 0.2) (layer "F.Cu") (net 17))
 (segment (start 144.215686 84.7) (end 157.984314 84.7) (width 0.2) (layer "F.Cu") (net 17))
 (segment (start 156.45 110.55) (end 156.45 111.65) (width 0.2) (layer "F.Cu") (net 17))
 (segment (start 143.25 94.5) (end 146.8 94.5) (width 0.2) (layer "F.Cu") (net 17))
 (segment (start 154.45 108.55) (end 156.45 110.55) (width 0.2) (layer "F.Cu") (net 17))
 (segment (start 146.8 94.5) (end 148.5 96.2) (width 0.2) (layer "F.Cu") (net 17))
 (via (at 143.25 94.5) (size 0.6) (drill 0.3) (layers "F.Cu" "B.Cu") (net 17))
 (via (at 148.5 96.2) (size 0.6) (drill 0.3) (layers "F.Cu" "B.Cu") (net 17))
 (via (at 154.45 108.55) (size 0.6) (drill 0.3) (layers "F.Cu" "B.Cu") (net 17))
 (segment (start 143.25 94.5) (end 141.75 94.5) (width 0.2) (layer "B.Cu") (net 17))
 (segment (start 148.5 96.2) (end 148.5 99) (width 0.2) (layer "B.Cu") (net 17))
 (segment (start 148.5 99) (end 154.45 104.95) (width 0.2) (layer "B.Cu") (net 17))
 (segment (start 154.45 104.95) (end 154.45 108.55) (width 0.2) (layer "B.Cu") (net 17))
 (segment (start 145.5925 97.1025) (end 150.6725 97.1025) (width 0.2) (layer "F.Cu") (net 12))
 (segment (start 140.85 95.6) (end 140.85 96.872793) (width 0.2) (layer "F.Cu") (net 12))
 (segment (start 142.079707 98.1025) (end 144.5925 98.1025) (width 0.2) (layer "F.Cu") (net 12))
 (segment (start 144.5925 98.1025) (end 145.5925 97.1025) (width 0.2) (layer "F.Cu") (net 12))
 (segment (start 140.85 96.872793) (end 142.079707 98.1025) (width 0.2) (layer "F.Cu") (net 12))
 (segment (start 139.75 94.5) (end 140.85 95.6) (width 0.2) (layer "F.Cu") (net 12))
 (segment (start 157.75 88.9) (end 159.55 90.7) (width 0.2) (layer "F.Cu") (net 16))
 (segment (start 146.45 92.6) (end 147.6 93.75) (width 0.2) (layer "F.Cu") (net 16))
 (segment (start 157.55 85.1) (end 157.75 85.3) (width 0.2) (layer "F.Cu") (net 16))
 (segment (start 157.75 85.3) (end 157.75 88.9) (width 0.2) (layer "F.Cu") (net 16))
 (segment (start 143.45 86.031372) (end 144.381372 85.1) (width 0.2) (layer "F.Cu") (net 16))
 (segment (start 143.45 92.4) (end 143.45 86.031372) (width 0.2) (layer "F.Cu") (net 16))
 (segment (start 143.65 92.6) (end 146.45 92.6) (width 0.2) (layer "F.Cu") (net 16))
 (segment (start 153.9 110.3) (end 153.9 111.6) (width 0.2) (layer "F.Cu") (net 16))
 (segment (start 143.65 92.6) (end 143.45 92.4) (width 0.2) (layer "F.Cu") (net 16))
 (segment (start 144.381372 85.1) (end 157.55 85.1) (width 0.2) (layer "F.Cu") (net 16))
 (segment (start 153.9 111.6) (end 153.95 111.65) (width 0.2) (layer "F.Cu") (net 16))
 (via (at 147.6 93.75) (size 0.6) (drill 0.3) (layers "F.Cu" "B.Cu") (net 16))
 (via (at 153.9 110.3) (size 0.6) (drill 0.3) (layers "F.Cu" "B.Cu") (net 16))
 (via (at 143.65 92.6) (size 0.6) (drill 0.3) (layers "F.Cu" "B.Cu") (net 16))
 (segment (start 143.65 92.6) (end 143.55 92.5) (width 0.2) (layer "B.Cu") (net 16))
 (segment (start 147.6 93.75) (end 147.6 98.75) (width 0.2) (layer "B.Cu") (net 16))
 (segment (start 153.85 105) (end 153.85 110.25) (width 0.2) (layer "B.Cu") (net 16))
 (segment (start 153.85 110.25) (end 153.9 110.3) (width 0.2) (layer "B.Cu") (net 16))
 (segment (start 143.55 92.5) (end 141.75 92.5) (width 0.2) (layer "B.Cu") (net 16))
 (segment (start 147.6 98.75) (end 153.85 105) (width 0.2) (layer "B.Cu") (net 16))
 (segment (start 158.85 85.051471) (end 159.801471 84.1) (width 0.2) (layer "F.Cu") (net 18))
 (segment (start 158.55 84.7) (end 158.15 84.3) (width 0.2) (layer "F.Cu") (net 18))
 (segment (start 159.55 86.7) (end 158.55 85.7) (width 0.2) (layer "F.Cu") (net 18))
 (segment (start 158.85 86) (end 158.85 85.051471) (width 0.2) (layer "F.Cu") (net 18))
 (segment (start 163.4 96.25) (end 161.45 98.2) (width 0.2) (layer "F.Cu") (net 18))
 (segment (start 161.45 98.2) (end 157.7 98.2) (width 0.2) (layer "F.Cu") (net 18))
 (segment (start 163.4 85.55) (end 163.4 96.25) (width 0.2) (layer "F.Cu") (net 18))
 (segment (start 144.05 84.3) (end 142.65 85.7) (width 0.2) (layer "F.Cu") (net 18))
 (segment (start 142.65 95.6) (end 141.75 96.5) (width 0.2) (layer "F.Cu") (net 18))
 (segment (start 161.95 84.1) (end 163.4 85.55) (width 0.2) (layer "F.Cu") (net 18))
 (segment (start 159.801471 84.1) (end 161.95 84.1) (width 0.2) (layer "F.Cu") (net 18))
 (segment (start 158.15 84.3) (end 144.05 84.3) (width 0.2) (layer "F.Cu") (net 18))
 (segment (start 157.7 110.35) (end 157.7 111.65) (width 0.2) (layer "F.Cu") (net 18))
 (segment (start 159.55 86.7) (end 158.85 86) (width 0.2) (layer "F.Cu") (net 18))
 (segment (start 158.55 85.7) (end 158.55 84.7) (width 0.2) (layer "F.Cu") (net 18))
 (segment (start 142.65 85.7) (end 142.65 95.6) (width 0.2) (layer "F.Cu") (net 18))
 (via (at 157.7 98.2) (size 0.6) (drill 0.3) (layers "F.Cu" "B.Cu") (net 18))
 (via (at 157.7 110.35) (size 0.6) (drill 0.3) (layers "F.Cu" "B.Cu") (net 18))
 (segment (start 157.7 98.2) (end 157.7 110.35) (width 0.2) (layer "B.Cu") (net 18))
 (segment (start 144.05 101.82) (end 144.05 106.9) (width 0.2) (layer "F.Cu") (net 3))
 (segment (start 142.1 95.5) (end 144.05 97.45) (width 0.2) (layer "B.Cu") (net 3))
 (segment (start 140.75 95) (end 141.25 95.5) (width 0.2) (layer "B.Cu") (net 3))
 (segment (start 141.75 88.5) (end 140.75 89.5) (width 0.2) (layer "B.Cu") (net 3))
 (segment (start 141.25 95.5) (end 142.1 95.5) (width 0.2) (layer "B.Cu") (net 3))
 (segment (start 144.05 97.45) (end 144.05 101.82) (width 0.2) (layer "B.Cu") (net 3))
 (segment (start 140.75 89.5) (end 140.75 95) (width 0.2) (layer "B.Cu") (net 3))
 (segment (start 163 95.25) (end 161.55 96.7) (width 0.2) (layer "F.Cu") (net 7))
 (segment (start 161.915686 84.7) (end 163 85.784314) (width 0.2) (layer "F.Cu") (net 7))
 (segment (start 139.75 86.5) (end 138.05 88.2) (width 0.2) (layer "F.Cu") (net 7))
 (segment (start 160.2 84.7) (end 161.915686 84.7) (width 0.2) (layer "F.Cu") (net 7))
 (segment (start 139.3 99.95) (end 139.3 111.65) (width 0.2) (layer "F.Cu") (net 7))
 (segment (start 138.05 88.2) (end 138.05 98.7) (width 0.2) (layer "F.Cu") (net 7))
 (segment (start 163 85.784314) (end 163 95.25) (width 0.2) (layer "F.Cu") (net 7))
 (segment (start 138.05 98.7) (end 139.3 99.95) (width 0.2) (layer "F.Cu") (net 7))
 (via (at 160.2 84.7) (size 0.6) (drill 0.3) (layers "F.Cu" "B.Cu") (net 7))
 (segment (start 139.75 85.651472) (end 139.75 86.5) (width 0.2) (layer "B.Cu") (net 7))
 (segment (start 140.701472 84.7) (end 139.75 85.651472) (width 0.2) (layer "B.Cu") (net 7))
 (segment (start 160.2 84.7) (end 140.701472 84.7) (width 0.2) (layer "B.Cu") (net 7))
 (segment (start 132.65 100.58) (end 133.89 101.82) (width 0.2) (layer "B.Cu") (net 5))
 (segment (start 160.565686 93.7) (end 161.95 93.7) (width 0.2) (layer "B.Cu") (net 5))
 (segment (start 159.565686 94.7) (end 160.565686 93.7) (width 0.2) (layer "B.Cu") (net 5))
 (segment (start 132.65 86.3) (end 132.65 100.58) (width 0.2) (layer "B.Cu") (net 5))
 (segment (start 160.448529 84.1) (end 134.85 84.1) (width 0.2) (layer "B.Cu") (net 5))
 (segment (start 134.85 84.1) (end 132.65 86.3) (width 0.2) (layer "B.Cu") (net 5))
 (segment (start 162.55 86.201471) (end 160.448529 84.1) (width 0.2) (layer "B.Cu") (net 5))
 (segment (start 162.55 93.1) (end 162.55 86.201471) (width 0.2) (layer "B.Cu") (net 5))
 (segment (start 159.55 94.7) (end 159.565686 94.7) (width 0.2) (layer "B.Cu") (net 5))
 (segment (start 161.95 93.7) (end 162.55 93.1) (width 0.2) (layer "B.Cu") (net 5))
 (segment (start 158.1 92.75) (end 158.1 92.3) (width 0.2) (layer "F.Cu") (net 14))
 (segment (start 160 93.7) (end 159.05 93.7) (width 0.2) (layer "F.Cu") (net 14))
 (segment (start 160.55 89.7) (end 160.55 93.15) (width 0.2) (layer "F.Cu") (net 14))
 (segment (start 159.05 93.7) (end 158.1 92.75) (width 0.2) (layer "F.Cu") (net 14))
 (segment (start 160.55 93.15) (end 160 93.7) (width 0.2) (layer "F.Cu") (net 14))
 (segment (start 161.55 88.7) (end 160.55 89.7) (width 0.2) (layer "F.Cu") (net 14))
 (via (at 158.1 92.3) (size 0.6) (drill 0.3) (layers "F.Cu" "B.Cu") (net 14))
 (segment (start 158.1 92.3) (end 155.4 92.3) (width 0.2) (layer "B.Cu") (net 14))
 (segment (start 153.7 90.6) (end 153.7 87.5) (width 0.2) (layer "B.Cu") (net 14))
 (segment (start 153.7 87.5) (end 153.1425 86.9425) (width 0.2) (layer "B.Cu") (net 14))
 (segment (start 153.1425 86.9425) (end 150.6725 86.9425) (width 0.2) (layer "B.Cu") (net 14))
 (segment (start 155.4 92.3) (end 153.7 90.6) (width 0.2) (layer "B.Cu") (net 14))
 (segment (start 149.9 111.1) (end 150.9 111.1) (width 0.2) (layer "F.Cu") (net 6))
 (segment (start 136.8 111.65) (end 136.2 111.65) (width 0.2) (layer "F.Cu") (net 6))
 (segment (start 161.7 104.8) (end 163.6 104.8) (width 0.2) (layer "F.Cu") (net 6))
 (segment (start 161.1 109.65) (end 161.1 106.75) (width 0.2) (layer "F.Cu") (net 6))
 (segment (start 161.55 104.95) (end 161.7 104.8) (width 0.2) (layer "F.Cu") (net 6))
 (segment (start 136.2 111.65) (end 135.6 111.05) (width 0.2) (layer "F.Cu") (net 6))
 (segment (start 150.9 111.1) (end 151.45 111.65) (width 0.2) (layer "F.Cu") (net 6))
 (via (at 161.55 104.95) (size 0.6) (drill 0.3) (layers "F.Cu" "B.Cu") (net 6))
 (via (at 135.6 111.05) (size 0.6) (drill 0.3) (layers "F.Cu" "B.Cu") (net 6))
 (via (at 149.9 111.1) (size 0.6) (drill 0.3) (layers "F.Cu" "B.Cu") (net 6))
 (via (at 161.1 106.75) (size 0.6) (drill 0.3) (layers "F.Cu" "B.Cu") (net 6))
 (via (at 161.1 109.65) (size 0.6) (drill 0.3) (layers "F.Cu" "B.Cu") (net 6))
 (segment (start 149.85 111.05) (end 149.9 111.1) (width 0.2) (layer "B.Cu") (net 6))
 (segment (start 159.7 111.1) (end 149.9 111.1) (width 0.2) (layer "B.Cu") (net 6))
 (segment (start 135.6 111.05) (end 149.85 111.05) (width 0.2) (layer "B.Cu") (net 6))
 (segment (start 161.1 105.4) (end 161.55 104.95) (width 0.2) (layer "B.Cu") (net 6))
 (segment (start 161.1 109.7) (end 159.7 111.1) (width 0.2) (layer "B.Cu") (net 6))
 (segment (start 161.1 109.65) (end 161.1 109.7) (width 0.2) (layer "B.Cu") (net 6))
 (segment (start 161.1 106.75) (end 161.1 105.4) (width 0.2) (layer "B.Cu") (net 6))
 (segment (start 140.55 110.35) (end 140.55 111.65) (width 0.2) (layer "F.Cu") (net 1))
 (segment (start 140.2 110) (end 140.55 110.35) (width 0.2) (layer "F.Cu") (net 1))
 (via (at 140.2 110) (size 0.6) (drill 0.3) (layers "F.Cu" "B.Cu") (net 1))
 (segment (start 133.89 106.9) (end 136.99 110) (width 0.2) (layer "B.Cu") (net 1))
 (segment (start 136.99 110) (end 140.2 110) (width 0.2) (layer "B.Cu") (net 1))
 (segment (start 145.5925 86.9425) (end 151.2 92.55) (width 0.2) (layer "F.Cu") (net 10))
 (segment (start 155.15 111.6) (end 155.2 111.65) (width 0.2) (layer "F.Cu") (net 10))
 (segment (start 151.2 92.55) (end 151.2 94.95) (width 0.2) (layer "F.Cu") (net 10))
 (segment (start 155.15 110.4) (end 155.15 111.6) (width 0.2) (layer "F.Cu") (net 10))
 (via (at 155.15 110.4) (size 0.6) (drill 0.3) (layers "F.Cu" "B.Cu") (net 10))
 (via (at 151.2 94.95) (size 0.6) (drill 0.3) (layers "F.Cu" "B.Cu") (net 10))
 (segment (start 155.15 98.9) (end 155.15 110.4) (width 0.2) (layer "B.Cu") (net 10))
 (segment (start 151.2 94.95) (end 155.15 98.9) (width 0.2) (layer "B.Cu") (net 10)))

